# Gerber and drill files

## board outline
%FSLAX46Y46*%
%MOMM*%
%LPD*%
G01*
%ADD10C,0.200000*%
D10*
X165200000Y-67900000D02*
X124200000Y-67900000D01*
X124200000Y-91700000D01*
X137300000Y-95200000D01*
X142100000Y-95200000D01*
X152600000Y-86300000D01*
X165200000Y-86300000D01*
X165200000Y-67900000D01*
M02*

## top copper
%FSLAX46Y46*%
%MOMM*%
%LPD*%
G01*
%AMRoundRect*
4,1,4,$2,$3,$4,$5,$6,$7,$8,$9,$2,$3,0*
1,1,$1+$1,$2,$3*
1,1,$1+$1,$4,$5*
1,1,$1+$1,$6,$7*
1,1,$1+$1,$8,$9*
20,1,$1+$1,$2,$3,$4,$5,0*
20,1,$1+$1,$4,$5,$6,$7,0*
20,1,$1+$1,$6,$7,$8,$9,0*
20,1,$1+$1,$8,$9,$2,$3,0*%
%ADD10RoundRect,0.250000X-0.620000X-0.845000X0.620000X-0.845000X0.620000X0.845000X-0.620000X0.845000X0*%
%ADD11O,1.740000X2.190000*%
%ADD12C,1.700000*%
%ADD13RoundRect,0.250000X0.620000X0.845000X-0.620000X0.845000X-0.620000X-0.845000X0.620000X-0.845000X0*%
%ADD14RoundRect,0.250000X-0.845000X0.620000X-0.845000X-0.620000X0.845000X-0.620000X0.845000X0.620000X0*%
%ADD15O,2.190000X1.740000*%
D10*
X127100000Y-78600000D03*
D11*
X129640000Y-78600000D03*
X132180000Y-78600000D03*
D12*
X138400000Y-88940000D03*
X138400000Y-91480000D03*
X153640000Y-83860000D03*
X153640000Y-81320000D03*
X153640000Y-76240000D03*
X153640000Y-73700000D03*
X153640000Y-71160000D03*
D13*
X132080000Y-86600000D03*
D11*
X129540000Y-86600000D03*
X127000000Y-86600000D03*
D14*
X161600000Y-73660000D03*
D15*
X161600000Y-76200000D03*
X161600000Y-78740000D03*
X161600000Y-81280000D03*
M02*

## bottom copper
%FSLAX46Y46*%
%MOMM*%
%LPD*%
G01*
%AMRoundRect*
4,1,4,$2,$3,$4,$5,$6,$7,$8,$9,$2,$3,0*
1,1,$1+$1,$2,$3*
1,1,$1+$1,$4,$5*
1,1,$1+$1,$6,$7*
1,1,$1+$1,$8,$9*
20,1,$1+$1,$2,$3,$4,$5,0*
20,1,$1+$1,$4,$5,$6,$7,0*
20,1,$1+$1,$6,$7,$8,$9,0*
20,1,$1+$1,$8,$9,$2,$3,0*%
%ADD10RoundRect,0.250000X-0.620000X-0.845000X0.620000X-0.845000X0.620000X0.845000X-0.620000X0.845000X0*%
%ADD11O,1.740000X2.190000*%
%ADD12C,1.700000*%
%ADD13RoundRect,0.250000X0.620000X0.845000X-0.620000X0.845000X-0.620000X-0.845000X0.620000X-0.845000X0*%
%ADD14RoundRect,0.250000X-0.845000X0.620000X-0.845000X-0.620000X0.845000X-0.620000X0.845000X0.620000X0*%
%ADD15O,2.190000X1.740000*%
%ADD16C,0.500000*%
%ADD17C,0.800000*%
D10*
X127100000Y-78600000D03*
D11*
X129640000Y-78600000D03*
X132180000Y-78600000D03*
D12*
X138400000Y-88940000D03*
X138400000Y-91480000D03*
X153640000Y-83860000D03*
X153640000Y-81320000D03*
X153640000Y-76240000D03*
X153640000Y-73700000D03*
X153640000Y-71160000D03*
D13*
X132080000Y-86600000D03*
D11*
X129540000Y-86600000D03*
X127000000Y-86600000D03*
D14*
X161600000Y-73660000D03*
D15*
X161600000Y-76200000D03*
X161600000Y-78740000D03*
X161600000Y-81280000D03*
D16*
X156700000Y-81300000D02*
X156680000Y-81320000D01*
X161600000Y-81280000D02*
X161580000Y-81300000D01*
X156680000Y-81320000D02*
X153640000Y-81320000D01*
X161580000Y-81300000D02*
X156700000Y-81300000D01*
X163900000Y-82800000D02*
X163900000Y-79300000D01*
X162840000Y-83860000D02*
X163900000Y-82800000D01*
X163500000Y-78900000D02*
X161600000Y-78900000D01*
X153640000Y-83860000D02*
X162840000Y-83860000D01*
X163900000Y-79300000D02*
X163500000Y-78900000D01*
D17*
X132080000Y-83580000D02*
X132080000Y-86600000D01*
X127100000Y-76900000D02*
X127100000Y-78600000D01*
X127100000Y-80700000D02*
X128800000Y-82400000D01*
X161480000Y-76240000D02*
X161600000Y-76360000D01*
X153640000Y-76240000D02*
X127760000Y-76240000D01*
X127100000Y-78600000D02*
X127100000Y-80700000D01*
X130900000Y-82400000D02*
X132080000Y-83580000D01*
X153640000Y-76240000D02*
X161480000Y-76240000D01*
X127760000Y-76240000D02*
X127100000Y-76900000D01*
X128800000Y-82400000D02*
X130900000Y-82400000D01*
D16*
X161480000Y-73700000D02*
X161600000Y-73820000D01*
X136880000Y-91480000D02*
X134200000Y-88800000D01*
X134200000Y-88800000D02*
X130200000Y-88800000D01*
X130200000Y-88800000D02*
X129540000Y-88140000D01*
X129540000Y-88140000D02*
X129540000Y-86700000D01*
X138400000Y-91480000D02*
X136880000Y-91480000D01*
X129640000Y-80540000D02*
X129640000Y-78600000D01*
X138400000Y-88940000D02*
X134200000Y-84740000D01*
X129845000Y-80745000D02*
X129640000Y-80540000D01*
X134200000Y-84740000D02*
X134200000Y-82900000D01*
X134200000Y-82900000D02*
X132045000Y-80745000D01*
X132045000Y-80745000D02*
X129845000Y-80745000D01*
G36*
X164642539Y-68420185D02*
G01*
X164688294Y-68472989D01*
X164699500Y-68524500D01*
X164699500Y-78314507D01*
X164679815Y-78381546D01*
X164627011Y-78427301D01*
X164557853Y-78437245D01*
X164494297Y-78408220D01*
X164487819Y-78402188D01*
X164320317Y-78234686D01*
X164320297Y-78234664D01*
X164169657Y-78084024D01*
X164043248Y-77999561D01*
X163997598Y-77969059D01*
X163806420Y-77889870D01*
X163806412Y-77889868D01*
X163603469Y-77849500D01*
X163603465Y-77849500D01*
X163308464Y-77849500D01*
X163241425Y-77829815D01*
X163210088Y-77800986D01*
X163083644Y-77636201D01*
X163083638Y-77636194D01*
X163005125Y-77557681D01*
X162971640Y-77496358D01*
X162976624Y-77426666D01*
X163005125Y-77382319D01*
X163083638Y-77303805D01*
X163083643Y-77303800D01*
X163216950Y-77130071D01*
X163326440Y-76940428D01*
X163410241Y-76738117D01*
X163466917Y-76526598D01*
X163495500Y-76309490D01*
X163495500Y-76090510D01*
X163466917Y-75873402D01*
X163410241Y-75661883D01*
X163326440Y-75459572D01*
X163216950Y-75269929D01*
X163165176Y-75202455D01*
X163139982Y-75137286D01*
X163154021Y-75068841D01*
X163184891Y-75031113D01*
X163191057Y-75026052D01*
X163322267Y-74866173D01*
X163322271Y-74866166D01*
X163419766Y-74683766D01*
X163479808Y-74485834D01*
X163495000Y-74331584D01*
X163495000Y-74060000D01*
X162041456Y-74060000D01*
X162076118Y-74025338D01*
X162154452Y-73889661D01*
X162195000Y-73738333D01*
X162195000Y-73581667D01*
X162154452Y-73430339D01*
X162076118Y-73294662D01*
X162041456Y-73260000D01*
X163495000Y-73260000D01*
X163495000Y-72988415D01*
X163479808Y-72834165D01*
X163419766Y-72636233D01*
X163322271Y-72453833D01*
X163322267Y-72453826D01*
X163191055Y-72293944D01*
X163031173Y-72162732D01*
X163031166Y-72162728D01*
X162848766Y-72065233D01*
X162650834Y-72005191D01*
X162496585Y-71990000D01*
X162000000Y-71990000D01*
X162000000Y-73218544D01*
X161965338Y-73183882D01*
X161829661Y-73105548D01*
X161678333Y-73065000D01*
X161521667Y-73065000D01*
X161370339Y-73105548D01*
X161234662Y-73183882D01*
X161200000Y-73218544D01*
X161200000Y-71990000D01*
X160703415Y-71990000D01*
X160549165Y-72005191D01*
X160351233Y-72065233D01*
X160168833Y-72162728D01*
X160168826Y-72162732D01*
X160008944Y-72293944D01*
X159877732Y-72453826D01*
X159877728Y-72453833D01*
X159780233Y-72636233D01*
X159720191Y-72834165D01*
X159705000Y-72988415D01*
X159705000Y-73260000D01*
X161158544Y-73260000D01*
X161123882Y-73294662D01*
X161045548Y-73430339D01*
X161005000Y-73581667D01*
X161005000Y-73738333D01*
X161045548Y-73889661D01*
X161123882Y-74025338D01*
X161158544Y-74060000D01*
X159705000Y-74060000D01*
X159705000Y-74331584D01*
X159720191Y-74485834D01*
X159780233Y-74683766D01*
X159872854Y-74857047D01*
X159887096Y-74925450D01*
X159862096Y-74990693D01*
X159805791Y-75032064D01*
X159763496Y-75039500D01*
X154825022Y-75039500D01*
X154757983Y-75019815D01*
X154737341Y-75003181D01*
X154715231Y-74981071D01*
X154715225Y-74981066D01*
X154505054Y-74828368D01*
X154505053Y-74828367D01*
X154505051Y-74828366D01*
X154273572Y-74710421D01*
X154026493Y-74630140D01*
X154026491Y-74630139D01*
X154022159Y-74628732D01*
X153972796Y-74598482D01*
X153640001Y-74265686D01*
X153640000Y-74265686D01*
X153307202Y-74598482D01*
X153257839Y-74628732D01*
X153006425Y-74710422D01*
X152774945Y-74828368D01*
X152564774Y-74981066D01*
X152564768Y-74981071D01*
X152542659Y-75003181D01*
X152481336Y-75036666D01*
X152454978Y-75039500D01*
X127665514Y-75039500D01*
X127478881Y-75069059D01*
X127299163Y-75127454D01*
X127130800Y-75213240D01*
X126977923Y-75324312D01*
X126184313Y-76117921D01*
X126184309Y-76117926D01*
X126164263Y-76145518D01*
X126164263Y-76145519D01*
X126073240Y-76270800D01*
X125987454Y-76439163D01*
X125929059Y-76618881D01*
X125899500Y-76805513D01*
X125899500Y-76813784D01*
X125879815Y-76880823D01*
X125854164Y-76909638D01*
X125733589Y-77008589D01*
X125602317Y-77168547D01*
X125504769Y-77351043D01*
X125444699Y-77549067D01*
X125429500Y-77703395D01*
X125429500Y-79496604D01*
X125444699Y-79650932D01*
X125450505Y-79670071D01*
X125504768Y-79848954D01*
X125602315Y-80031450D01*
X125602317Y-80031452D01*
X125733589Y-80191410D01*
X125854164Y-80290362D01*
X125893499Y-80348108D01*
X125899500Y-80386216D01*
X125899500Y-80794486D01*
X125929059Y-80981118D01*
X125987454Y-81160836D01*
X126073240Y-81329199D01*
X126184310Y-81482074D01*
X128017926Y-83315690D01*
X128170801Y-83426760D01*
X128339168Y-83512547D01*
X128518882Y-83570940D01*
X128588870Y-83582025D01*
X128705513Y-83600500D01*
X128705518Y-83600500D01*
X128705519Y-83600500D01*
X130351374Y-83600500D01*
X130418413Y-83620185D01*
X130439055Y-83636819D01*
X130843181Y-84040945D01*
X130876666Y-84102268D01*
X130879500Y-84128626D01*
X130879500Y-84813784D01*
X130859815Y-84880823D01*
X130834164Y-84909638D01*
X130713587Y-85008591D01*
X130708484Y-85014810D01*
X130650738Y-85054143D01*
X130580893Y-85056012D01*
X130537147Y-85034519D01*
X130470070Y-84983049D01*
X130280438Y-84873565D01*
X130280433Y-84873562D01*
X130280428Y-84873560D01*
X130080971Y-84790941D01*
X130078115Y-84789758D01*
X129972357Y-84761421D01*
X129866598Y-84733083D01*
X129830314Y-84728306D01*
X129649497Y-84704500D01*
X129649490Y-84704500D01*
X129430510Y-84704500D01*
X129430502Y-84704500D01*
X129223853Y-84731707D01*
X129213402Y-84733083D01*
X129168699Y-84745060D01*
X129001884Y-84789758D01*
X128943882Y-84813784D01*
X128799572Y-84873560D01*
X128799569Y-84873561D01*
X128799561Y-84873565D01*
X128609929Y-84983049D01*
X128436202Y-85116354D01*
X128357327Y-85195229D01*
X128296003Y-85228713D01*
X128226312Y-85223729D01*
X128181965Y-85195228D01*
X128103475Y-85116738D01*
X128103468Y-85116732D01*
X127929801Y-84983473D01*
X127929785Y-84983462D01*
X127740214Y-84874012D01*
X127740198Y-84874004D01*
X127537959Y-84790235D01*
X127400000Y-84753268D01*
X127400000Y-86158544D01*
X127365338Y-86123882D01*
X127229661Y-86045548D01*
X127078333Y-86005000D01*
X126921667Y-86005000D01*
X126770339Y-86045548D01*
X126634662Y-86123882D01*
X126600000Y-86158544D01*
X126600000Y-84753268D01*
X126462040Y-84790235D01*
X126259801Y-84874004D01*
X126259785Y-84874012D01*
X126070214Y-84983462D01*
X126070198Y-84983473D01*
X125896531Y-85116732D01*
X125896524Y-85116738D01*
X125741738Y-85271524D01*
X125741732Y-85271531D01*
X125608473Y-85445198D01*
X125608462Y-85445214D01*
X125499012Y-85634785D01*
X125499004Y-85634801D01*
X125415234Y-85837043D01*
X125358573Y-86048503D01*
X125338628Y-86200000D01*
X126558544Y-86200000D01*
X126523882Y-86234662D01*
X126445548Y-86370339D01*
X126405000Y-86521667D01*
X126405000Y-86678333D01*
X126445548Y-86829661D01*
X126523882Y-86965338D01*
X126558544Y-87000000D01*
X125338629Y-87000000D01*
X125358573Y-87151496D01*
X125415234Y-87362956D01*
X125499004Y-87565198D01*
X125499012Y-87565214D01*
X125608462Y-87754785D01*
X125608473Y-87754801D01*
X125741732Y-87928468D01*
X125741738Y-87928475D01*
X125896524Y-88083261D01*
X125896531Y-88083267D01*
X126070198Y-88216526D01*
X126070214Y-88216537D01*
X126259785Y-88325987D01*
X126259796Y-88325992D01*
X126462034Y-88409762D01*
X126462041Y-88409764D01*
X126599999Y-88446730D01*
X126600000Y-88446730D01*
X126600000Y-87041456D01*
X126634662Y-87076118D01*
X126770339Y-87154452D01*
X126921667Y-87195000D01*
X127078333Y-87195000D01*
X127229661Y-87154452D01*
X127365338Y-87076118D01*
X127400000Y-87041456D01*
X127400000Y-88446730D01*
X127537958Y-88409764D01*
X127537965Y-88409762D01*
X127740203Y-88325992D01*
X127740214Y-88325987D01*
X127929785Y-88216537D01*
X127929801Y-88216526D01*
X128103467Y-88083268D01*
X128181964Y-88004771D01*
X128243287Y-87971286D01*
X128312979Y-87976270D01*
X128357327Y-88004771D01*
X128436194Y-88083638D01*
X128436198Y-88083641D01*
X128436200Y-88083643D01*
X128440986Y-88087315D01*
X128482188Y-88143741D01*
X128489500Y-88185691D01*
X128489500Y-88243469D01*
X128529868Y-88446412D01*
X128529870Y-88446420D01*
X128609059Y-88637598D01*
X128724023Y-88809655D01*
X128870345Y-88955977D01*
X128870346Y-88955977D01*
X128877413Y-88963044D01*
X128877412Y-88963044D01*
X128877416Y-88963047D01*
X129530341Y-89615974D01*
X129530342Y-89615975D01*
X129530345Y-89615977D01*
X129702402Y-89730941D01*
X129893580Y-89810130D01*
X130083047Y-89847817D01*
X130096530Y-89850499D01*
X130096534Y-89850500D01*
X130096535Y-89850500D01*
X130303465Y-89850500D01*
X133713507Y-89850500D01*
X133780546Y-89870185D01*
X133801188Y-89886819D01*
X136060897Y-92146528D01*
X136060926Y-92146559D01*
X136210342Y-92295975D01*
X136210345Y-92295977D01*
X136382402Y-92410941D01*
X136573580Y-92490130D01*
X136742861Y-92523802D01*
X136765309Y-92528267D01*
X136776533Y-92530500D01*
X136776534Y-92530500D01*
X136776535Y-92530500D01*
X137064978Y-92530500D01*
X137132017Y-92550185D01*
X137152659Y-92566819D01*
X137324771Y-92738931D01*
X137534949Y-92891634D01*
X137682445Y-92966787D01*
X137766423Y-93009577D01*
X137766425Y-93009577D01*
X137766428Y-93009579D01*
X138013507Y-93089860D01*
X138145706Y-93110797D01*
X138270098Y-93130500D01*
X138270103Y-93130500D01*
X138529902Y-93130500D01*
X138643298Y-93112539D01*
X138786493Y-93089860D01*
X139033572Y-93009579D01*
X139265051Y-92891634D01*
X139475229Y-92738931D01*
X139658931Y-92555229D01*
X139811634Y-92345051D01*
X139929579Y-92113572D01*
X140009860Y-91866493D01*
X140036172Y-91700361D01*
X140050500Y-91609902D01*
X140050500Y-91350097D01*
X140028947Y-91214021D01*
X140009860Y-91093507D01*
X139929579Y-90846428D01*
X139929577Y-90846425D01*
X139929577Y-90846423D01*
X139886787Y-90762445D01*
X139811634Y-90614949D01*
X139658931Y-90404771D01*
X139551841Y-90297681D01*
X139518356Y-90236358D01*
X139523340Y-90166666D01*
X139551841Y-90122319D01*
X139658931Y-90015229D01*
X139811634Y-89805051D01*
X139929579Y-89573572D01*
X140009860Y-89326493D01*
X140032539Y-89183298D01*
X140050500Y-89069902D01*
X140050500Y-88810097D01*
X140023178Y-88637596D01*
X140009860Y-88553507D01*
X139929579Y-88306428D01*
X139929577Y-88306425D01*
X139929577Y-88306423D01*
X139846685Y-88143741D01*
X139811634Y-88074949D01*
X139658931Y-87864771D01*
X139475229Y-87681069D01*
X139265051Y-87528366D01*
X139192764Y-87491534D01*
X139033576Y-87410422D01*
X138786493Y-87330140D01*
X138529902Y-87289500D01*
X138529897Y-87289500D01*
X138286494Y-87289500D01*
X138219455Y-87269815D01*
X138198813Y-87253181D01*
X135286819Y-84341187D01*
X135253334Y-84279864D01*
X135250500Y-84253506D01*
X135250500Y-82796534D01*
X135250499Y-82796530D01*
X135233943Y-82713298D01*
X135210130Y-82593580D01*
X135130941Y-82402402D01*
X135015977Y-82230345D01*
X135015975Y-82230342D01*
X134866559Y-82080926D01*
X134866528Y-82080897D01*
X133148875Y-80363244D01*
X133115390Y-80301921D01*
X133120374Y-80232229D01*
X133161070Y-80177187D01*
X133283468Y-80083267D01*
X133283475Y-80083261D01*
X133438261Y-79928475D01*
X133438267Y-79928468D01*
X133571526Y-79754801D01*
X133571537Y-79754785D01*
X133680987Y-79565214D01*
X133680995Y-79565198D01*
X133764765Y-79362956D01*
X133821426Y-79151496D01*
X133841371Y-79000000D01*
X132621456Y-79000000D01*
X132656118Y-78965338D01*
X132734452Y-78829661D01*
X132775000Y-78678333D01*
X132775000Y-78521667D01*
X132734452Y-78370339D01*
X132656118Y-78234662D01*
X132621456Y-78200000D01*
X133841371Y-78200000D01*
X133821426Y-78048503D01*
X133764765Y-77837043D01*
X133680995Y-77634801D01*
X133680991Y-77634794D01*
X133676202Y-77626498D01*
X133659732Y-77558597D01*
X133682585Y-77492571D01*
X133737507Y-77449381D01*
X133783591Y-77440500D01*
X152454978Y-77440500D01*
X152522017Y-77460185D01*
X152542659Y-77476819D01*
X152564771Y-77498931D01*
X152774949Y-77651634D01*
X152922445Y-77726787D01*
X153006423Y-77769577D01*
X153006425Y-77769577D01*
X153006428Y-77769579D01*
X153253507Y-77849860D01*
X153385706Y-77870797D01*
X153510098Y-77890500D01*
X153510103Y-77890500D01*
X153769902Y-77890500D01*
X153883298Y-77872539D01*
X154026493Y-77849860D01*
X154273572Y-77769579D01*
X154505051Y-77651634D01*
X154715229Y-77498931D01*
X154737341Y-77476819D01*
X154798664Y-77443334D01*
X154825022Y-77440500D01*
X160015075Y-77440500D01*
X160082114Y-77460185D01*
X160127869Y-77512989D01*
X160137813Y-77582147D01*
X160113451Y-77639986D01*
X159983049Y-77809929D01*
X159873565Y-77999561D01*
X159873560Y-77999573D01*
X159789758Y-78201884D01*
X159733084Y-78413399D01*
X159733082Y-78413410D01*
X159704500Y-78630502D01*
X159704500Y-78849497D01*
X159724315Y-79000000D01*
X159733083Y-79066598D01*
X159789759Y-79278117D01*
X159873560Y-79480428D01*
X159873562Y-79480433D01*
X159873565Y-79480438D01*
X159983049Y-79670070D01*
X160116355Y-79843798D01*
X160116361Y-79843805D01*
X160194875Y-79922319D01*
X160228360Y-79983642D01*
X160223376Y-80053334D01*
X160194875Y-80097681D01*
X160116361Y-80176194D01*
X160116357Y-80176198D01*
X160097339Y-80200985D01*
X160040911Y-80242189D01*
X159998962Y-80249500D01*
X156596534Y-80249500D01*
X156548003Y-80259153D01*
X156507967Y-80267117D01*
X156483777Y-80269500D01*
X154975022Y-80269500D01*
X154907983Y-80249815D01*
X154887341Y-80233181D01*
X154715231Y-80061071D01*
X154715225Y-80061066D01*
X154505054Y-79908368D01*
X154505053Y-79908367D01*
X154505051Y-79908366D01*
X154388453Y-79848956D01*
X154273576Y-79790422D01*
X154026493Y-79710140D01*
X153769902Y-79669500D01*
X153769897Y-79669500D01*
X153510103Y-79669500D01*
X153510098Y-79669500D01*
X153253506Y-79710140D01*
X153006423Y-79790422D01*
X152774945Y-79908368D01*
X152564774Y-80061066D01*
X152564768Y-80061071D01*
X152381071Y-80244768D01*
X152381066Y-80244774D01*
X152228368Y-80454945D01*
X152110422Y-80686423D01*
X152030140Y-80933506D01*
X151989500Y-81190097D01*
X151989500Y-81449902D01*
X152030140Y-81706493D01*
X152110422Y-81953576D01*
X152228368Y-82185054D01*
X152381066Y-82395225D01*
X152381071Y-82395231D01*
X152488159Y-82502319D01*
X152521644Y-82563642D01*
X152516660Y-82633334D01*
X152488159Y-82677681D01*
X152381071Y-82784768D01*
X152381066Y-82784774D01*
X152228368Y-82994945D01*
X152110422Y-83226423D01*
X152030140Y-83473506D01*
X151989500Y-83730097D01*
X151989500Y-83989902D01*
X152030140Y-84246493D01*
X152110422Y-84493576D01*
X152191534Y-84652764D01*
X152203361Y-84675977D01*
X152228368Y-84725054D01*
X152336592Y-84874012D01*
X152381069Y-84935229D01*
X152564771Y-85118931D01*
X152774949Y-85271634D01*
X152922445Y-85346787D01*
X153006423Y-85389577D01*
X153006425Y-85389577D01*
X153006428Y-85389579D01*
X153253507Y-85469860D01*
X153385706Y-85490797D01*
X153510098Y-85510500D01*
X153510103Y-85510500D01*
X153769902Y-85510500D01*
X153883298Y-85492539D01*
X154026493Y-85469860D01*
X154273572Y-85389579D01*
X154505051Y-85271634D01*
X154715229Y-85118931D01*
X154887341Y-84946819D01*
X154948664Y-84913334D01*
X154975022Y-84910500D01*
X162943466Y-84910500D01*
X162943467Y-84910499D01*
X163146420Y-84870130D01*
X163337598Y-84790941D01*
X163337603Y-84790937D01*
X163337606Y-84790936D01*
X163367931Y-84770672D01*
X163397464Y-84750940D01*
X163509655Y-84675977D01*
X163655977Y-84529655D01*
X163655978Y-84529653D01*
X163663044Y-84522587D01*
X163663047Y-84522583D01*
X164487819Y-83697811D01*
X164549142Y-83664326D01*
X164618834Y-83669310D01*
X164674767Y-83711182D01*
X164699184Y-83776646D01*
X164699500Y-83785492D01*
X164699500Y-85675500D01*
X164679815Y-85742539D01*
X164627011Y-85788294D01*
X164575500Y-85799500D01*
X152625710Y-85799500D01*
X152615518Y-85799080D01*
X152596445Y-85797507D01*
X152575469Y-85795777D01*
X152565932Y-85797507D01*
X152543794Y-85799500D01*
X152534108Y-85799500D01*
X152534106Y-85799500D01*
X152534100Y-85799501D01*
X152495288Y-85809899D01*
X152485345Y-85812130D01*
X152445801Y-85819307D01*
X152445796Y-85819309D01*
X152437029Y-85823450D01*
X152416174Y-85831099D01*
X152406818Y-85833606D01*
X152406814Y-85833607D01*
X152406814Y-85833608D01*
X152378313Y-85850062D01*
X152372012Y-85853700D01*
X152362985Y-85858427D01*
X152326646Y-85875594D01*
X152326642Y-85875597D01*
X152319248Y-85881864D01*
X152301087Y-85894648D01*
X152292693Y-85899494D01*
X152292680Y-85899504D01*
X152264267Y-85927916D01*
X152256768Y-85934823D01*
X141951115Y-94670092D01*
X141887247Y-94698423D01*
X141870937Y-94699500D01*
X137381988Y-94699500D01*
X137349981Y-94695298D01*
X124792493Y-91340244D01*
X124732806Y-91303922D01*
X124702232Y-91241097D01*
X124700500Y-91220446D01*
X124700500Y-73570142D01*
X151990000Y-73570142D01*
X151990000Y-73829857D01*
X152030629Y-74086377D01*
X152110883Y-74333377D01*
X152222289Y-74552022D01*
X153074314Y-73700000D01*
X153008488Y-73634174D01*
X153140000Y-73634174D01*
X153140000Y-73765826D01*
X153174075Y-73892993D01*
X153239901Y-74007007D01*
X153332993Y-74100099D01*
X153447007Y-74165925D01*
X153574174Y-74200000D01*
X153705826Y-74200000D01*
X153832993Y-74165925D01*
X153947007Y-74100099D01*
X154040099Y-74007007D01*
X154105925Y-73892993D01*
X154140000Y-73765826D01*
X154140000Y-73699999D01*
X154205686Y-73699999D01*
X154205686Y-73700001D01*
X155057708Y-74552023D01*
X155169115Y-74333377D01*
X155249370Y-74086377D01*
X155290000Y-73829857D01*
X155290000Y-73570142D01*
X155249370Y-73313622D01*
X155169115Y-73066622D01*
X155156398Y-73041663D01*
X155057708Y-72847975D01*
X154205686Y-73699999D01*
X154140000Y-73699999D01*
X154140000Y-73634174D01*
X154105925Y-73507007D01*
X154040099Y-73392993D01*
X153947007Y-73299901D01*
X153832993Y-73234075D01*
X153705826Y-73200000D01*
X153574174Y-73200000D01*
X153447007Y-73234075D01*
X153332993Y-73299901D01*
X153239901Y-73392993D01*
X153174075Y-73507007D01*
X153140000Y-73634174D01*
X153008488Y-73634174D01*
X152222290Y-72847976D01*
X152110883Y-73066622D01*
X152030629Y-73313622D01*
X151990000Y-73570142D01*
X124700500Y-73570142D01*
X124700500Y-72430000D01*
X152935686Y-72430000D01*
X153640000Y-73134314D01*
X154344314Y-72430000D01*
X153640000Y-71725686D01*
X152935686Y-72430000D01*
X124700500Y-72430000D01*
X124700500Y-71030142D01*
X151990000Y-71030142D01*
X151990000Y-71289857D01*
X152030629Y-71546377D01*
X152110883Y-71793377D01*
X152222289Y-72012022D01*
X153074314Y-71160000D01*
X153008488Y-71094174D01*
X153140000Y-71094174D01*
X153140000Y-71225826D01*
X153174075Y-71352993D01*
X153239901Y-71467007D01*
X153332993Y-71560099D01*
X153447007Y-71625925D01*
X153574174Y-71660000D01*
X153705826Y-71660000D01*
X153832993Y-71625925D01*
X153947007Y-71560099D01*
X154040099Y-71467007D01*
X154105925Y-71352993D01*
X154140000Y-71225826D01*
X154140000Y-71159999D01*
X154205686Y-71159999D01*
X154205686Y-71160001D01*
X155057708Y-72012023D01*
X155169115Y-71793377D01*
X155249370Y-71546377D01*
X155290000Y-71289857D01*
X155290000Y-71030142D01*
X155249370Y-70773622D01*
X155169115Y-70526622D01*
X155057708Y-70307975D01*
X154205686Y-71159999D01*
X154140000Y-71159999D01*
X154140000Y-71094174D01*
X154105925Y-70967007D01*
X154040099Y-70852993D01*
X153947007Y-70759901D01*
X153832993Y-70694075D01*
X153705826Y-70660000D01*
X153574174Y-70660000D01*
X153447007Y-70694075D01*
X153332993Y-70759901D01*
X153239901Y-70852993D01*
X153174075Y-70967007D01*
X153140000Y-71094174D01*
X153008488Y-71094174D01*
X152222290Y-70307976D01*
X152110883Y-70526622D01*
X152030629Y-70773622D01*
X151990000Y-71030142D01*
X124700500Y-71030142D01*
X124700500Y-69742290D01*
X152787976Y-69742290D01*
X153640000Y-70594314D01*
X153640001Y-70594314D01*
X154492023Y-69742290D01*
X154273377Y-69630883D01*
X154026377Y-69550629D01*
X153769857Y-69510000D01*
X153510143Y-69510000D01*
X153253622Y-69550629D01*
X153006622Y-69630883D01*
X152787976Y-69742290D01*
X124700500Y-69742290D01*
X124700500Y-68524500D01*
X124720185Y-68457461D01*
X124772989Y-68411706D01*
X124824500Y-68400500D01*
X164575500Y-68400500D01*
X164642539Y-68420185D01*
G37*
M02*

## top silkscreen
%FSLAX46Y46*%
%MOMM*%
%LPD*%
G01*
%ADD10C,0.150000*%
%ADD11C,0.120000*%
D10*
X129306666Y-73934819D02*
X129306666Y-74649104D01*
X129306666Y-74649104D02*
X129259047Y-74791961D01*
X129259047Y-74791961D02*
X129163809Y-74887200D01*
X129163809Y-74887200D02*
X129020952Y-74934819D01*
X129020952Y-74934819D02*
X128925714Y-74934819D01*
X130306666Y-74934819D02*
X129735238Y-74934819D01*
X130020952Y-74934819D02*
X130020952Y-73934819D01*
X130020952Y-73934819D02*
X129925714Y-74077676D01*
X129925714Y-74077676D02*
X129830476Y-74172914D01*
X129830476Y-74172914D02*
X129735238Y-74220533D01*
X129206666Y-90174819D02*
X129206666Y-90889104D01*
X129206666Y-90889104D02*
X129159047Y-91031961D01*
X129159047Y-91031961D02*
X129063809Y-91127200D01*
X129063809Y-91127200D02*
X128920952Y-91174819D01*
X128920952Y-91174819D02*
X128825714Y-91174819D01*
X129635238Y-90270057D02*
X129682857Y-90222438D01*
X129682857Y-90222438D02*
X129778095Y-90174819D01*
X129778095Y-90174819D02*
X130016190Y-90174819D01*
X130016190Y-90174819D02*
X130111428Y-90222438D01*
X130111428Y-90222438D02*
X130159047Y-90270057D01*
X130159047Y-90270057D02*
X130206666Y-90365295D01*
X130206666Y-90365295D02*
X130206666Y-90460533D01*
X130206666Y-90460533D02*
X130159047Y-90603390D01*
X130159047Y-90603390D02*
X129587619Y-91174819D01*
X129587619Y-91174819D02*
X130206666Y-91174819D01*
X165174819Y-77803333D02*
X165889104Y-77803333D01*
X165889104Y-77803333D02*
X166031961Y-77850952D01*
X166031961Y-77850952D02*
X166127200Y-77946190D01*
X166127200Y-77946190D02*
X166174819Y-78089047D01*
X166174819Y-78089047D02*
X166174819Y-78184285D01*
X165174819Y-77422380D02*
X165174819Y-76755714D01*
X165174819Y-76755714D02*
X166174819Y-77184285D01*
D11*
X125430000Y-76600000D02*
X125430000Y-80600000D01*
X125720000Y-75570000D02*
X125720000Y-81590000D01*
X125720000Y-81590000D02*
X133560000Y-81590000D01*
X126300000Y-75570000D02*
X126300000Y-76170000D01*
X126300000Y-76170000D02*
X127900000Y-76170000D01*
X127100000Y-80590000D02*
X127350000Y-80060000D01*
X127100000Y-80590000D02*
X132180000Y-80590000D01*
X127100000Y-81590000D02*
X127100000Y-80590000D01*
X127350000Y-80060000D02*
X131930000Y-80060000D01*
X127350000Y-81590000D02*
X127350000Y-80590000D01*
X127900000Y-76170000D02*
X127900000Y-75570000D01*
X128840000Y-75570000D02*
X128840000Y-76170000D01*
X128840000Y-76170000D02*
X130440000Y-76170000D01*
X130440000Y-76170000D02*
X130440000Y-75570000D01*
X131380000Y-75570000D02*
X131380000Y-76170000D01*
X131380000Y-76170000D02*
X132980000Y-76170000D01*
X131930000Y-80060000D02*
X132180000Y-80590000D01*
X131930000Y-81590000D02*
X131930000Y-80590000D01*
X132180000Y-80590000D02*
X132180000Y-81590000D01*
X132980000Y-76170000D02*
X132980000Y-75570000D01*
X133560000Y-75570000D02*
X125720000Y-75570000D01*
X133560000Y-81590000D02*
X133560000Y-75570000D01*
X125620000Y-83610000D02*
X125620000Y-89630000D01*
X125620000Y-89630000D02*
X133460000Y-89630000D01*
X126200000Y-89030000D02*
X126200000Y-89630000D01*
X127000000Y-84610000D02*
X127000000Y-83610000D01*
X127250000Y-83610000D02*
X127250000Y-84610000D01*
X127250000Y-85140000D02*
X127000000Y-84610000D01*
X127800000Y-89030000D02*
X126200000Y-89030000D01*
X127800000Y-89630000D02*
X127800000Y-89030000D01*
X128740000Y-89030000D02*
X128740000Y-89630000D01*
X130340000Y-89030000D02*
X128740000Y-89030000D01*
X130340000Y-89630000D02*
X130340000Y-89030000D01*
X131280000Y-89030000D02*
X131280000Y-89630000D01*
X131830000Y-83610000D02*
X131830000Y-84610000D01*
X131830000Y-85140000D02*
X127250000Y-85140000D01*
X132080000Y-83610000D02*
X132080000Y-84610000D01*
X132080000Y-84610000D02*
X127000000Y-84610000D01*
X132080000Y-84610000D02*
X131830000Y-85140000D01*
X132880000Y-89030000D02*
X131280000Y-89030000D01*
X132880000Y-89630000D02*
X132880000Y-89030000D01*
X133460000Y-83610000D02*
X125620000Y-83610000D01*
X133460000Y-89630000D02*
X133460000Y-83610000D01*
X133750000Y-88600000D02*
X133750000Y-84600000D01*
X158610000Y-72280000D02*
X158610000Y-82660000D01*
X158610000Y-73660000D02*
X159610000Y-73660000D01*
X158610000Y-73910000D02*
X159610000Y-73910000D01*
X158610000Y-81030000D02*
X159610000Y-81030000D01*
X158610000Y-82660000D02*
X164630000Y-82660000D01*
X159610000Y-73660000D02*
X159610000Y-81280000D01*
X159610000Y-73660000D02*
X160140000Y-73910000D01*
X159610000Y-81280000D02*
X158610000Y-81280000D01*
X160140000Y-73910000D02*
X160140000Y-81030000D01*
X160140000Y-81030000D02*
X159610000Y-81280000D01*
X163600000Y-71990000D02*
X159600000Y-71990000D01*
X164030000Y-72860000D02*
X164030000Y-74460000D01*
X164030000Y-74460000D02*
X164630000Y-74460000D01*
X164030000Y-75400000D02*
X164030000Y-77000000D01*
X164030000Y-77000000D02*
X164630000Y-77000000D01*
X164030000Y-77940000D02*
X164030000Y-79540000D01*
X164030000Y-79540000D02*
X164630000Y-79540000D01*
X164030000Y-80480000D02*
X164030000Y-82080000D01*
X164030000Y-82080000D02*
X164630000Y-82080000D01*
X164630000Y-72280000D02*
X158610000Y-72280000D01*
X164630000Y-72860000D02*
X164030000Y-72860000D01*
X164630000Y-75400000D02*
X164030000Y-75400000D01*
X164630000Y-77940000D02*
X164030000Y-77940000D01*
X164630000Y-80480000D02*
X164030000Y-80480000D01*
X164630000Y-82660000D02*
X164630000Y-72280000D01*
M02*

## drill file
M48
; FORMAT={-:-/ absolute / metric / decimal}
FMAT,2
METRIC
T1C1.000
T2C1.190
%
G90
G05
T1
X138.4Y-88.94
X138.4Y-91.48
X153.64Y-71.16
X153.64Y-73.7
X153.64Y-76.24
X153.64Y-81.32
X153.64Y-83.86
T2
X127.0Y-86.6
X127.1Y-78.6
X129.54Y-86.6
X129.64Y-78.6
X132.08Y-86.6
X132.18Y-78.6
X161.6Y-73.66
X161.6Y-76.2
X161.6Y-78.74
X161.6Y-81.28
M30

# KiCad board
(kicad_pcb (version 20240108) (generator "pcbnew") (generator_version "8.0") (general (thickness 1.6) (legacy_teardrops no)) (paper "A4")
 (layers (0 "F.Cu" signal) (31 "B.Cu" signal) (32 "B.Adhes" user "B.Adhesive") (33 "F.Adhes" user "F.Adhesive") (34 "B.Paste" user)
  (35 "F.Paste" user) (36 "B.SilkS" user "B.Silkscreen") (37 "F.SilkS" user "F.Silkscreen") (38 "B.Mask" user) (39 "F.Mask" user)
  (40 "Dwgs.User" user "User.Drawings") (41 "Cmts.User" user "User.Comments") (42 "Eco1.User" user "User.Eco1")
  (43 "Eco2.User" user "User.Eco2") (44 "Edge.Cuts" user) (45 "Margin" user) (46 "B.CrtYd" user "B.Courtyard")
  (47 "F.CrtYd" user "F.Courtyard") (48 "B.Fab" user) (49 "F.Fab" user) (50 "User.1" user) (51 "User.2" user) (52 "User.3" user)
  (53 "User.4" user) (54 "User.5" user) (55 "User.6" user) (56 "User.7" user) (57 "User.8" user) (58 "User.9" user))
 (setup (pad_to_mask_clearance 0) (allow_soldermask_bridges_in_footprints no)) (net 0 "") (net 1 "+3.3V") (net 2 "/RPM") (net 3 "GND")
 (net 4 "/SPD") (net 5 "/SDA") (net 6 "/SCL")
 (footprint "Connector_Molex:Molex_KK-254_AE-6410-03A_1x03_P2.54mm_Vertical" (layer "F.Cu") (at 127.1 78.6)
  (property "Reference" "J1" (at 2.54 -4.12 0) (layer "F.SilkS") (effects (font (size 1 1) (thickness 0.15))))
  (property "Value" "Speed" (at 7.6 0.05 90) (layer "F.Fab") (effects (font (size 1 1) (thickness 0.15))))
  (fp_line (start -1.67 -2) (end -1.67 2) (stroke (width 0.12) (type solid)) (layer "F.SilkS"))
  (fp_line (start -1.38 -3.03) (end -1.38 2.99) (stroke (width 0.12) (type solid)) (layer "F.SilkS"))
  (fp_line (start -1.38 2.99) (end 6.46 2.99) (stroke (width 0.12) (type solid)) (layer "F.SilkS"))
  (fp_line (start -0.8 -3.03) (end -0.8 -2.43) (stroke (width 0.12) (type solid)) (layer "F.SilkS"))
  (fp_line (start -0.8 -2.43) (end 0.8 -2.43) (stroke (width 0.12) (type solid)) (layer "F.SilkS"))
  (fp_line (start 0 1.99) (end 0.25 1.46) (stroke (width 0.12) (type solid)) (layer "F.SilkS"))
  (fp_line (start 0 1.99) (end 5.08 1.99) (stroke (width 0.12) (type solid)) (layer "F.SilkS"))
  (fp_line (start 0 2.99) (end 0 1.99) (stroke (width 0.12) (type solid)) (layer "F.SilkS"))
  (fp_line (start 0.25 1.46) (end 4.83 1.46) (stroke (width 0.12) (type solid)) (layer "F.SilkS"))
  (fp_line (start 0.25 2.99) (end 0.25 1.99) (stroke (width 0.12) (type solid)) (layer "F.SilkS"))
  (fp_line (start 0.8 -2.43) (end 0.8 -3.03) (stroke (width 0.12) (type solid)) (layer "F.SilkS"))
  (fp_line (start 1.74 -3.03) (end 1.74 -2.43) (stroke (width 0.12) (type solid)) (layer "F.SilkS"))
  (fp_line (start 1.74 -2.43) (end 3.34 -2.43) (stroke (width 0.12) (type solid)) (layer "F.SilkS"))
  (fp_line (start 3.34 -2.43) (end 3.34 -3.03) (stroke (width 0.12) (type solid)) (layer "F.SilkS"))
  (fp_line (start 4.28 -3.03) (end 4.28 -2.43) (stroke (width 0.12) (type solid)) (layer "F.SilkS"))
  (fp_line (start 4.28 -2.43) (end 5.88 -2.43) (stroke (width 0.12) (type solid)) (layer "F.SilkS"))
  (fp_line (start 4.83 1.46) (end 5.08 1.99) (stroke (width 0.12) (type solid)) (layer "F.SilkS"))
  (fp_line (start 4.83 2.99) (end 4.83 1.99) (stroke (width 0.12) (type solid)) (layer "F.SilkS"))
  (fp_line (start 5.08 1.99) (end 5.08 2.99) (stroke (width 0.12) (type solid)) (layer "F.SilkS"))
  (fp_line (start 5.88 -2.43) (end 5.88 -3.03) (stroke (width 0.12) (type solid)) (layer "F.SilkS"))
  (fp_line (start 6.46 -3.03) (end -1.38 -3.03) (stroke (width 0.12) (type solid)) (layer "F.SilkS"))
  (fp_line (start 6.46 2.99) (end 6.46 -3.03) (stroke (width 0.12) (type solid)) (layer "F.SilkS"))
  (pad "1" thru_hole roundrect (at 0 0) (size 1.74 2.19) (drill 1.19) (layers "*.Cu" "*.Mask") (remove_unused_layers no)
   (roundrect_rratio 0.143678) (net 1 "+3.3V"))
  (pad "2" thru_hole oval (at 2.54 0) (size 1.74 2.19) (drill 1.19) (layers "*.Cu" "*.Mask") (remove_unused_layers no) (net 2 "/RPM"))
  (pad "3" thru_hole oval (at 5.08 0) (size 1.74 2.19) (drill 1.19) (layers "*.Cu" "*.Mask") (remove_unused_layers no) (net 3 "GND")))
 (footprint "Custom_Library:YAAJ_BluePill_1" (layer "F.Cu") (at 138.4 71.16)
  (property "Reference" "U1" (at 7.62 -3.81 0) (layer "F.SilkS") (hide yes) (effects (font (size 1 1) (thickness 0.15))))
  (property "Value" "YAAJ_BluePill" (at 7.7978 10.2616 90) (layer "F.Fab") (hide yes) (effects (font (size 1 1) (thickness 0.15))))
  (pad "8" thru_hole circle (at 0 17.78) (size 1.7 1.7) (drill 1) (layers "*.Cu" "*.Mask") (remove_unused_layers no) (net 2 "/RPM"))
  (pad "9" thru_hole circle (at 0 20.32) (size 1.7 1.7) (drill 1) (layers "*.Cu" "*.Mask") (remove_unused_layers no) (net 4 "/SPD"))
  (pad "35" thru_hole circle (at 15.24 12.7) (size 1.7 1.7) (drill 1) (layers "*.Cu" "*.Mask") (remove_unused_layers no) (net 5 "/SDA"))
  (pad "36" thru_hole circle (at 15.24 10.16) (size 1.7 1.7) (drill 1) (layers "*.Cu" "*.Mask") (remove_unused_layers no) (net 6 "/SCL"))
  (pad "38" thru_hole circle (at 15.24 5.08) (size 1.7 1.7) (drill 1) (layers "*.Cu" "*.Mask") (remove_unused_layers no) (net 1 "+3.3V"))
  (pad "39" thru_hole circle (at 15.24 2.54) (size 1.7 1.7) (drill 1) (layers "*.Cu" "*.Mask") (remove_unused_layers no) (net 3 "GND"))
  (pad "40" thru_hole circle (at 15.24 0) (size 1.7 1.7) (drill 1) (layers "*.Cu" "*.Mask") (remove_unused_layers no) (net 3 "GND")))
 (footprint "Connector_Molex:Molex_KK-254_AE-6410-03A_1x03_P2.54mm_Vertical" (layer "F.Cu") (at 132.08 86.6 180)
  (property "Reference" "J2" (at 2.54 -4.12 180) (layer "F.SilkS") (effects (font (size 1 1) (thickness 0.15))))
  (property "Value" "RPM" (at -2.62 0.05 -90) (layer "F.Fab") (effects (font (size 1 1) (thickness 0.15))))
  (fp_line (start 6.46 2.99) (end 6.46 -3.03) (stroke (width 0.12) (type solid)) (layer "F.SilkS"))
  (fp_line (start 6.46 -3.03) (end -1.38 -3.03) (stroke (width 0.12) (type solid)) (layer "F.SilkS"))
  (fp_line (start 5.88 -2.43) (end 5.88 -3.03) (stroke (width 0.12) (type solid)) (layer "F.SilkS"))
  (fp_line (start 5.08 1.99) (end 5.08 2.99) (stroke (width 0.12) (type solid)) (layer "F.SilkS"))
  (fp_line (start 4.83 2.99) (end 4.83 1.99) (stroke (width 0.12) (type solid)) (layer "F.SilkS"))
  (fp_line (start 4.83 1.46) (end 5.08 1.99) (stroke (width 0.12) (type solid)) (layer "F.SilkS"))
  (fp_line (start 4.28 -2.43) (end 5.88 -2.43) (stroke (width 0.12) (type solid)) (layer "F.SilkS"))
  (fp_line (start 4.28 -3.03) (end 4.28 -2.43) (stroke (width 0.12) (type solid)) (layer "F.SilkS"))
  (fp_line (start 3.34 -2.43) (end 3.34 -3.03) (stroke (width 0.12) (type solid)) (layer "F.SilkS"))
  (fp_line (start 1.74 -2.43) (end 3.34 -2.43) (stroke (width 0.12) (type solid)) (layer "F.SilkS"))
  (fp_line (start 1.74 -3.03) (end 1.74 -2.43) (stroke (width 0.12) (type solid)) (layer "F.SilkS"))
  (fp_line (start 0.8 -2.43) (end 0.8 -3.03) (stroke (width 0.12) (type solid)) (layer "F.SilkS"))
  (fp_line (start 0.25 2.99) (end 0.25 1.99) (stroke (width 0.12) (type solid)) (layer "F.SilkS"))
  (fp_line (start 0.25 1.46) (end 4.83 1.46) (stroke (width 0.12) (type solid)) (layer "F.SilkS"))
  (fp_line (start 0 2.99) (end 0 1.99) (stroke (width 0.12) (type solid)) (layer "F.SilkS"))
  (fp_line (start 0 1.99) (end 5.08 1.99) (stroke (width 0.12) (type solid)) (layer "F.SilkS"))
  (fp_line (start 0 1.99) (end 0.25 1.46) (stroke (width 0.12) (type solid)) (layer "F.SilkS"))
  (fp_line (start -0.8 -2.43) (end 0.8 -2.43) (stroke (width 0.12) (type solid)) (layer "F.SilkS"))
  (fp_line (start -0.8 -3.03) (end -0.8 -2.43) (stroke (width 0.12) (type solid)) (layer "F.SilkS"))
  (fp_line (start -1.38 2.99) (end 6.46 2.99) (stroke (width 0.12) (type solid)) (layer "F.SilkS"))
  (fp_line (start -1.38 -3.03) (end -1.38 2.99) (stroke (width 0.12) (type solid)) (layer "F.SilkS"))
  (fp_line (start -1.67 -2) (end -1.67 2) (stroke (width 0.12) (type solid)) (layer "F.SilkS"))
  (pad "1" thru_hole roundrect (at 0 0 180) (size 1.74 2.19) (drill 1.19) (layers "*.Cu" "*.Mask") (remove_unused_layers no)
   (roundrect_rratio 0.143678) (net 1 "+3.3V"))
  (pad "2" thru_hole oval (at 2.54 0 180) (size 1.74 2.19) (drill 1.19) (layers "*.Cu" "*.Mask") (remove_unused_layers no) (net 4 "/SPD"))
  (pad "3" thru_hole oval (at 5.08 0 180) (size 1.74 2.19) (drill 1.19) (layers "*.Cu" "*.Mask") (remove_unused_layers no) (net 3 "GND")))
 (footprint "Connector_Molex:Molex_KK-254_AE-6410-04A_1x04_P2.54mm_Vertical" (layer "F.Cu") (at 161.6 73.66 -90)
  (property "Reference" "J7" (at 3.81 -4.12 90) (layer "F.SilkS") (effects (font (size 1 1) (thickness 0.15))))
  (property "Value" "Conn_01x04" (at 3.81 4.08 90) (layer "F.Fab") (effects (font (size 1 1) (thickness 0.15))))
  (fp_line (start -1.38 2.99) (end 9 2.99) (stroke (width 0.12) (type solid)) (layer "F.SilkS"))
  (fp_line (start 0 2.99) (end 0 1.99) (stroke (width 0.12) (type solid)) (layer "F.SilkS"))
  (fp_line (start 0.25 2.99) (end 0.25 1.99) (stroke (width 0.12) (type solid)) (layer "F.SilkS"))
  (fp_line (start 7.37 2.99) (end 7.37 1.99) (stroke (width 0.12) (type solid)) (layer "F.SilkS"))
  (fp_line (start 9 2.99) (end 9 -3.03) (stroke (width 0.12) (type solid)) (layer "F.SilkS"))
  (fp_line (start 0 1.99) (end 7.62 1.99) (stroke (width 0.12) (type solid)) (layer "F.SilkS"))
  (fp_line (start 0 1.99) (end 0.25 1.46) (stroke (width 0.12) (type solid)) (layer "F.SilkS"))
  (fp_line (start 7.62 1.99) (end 7.62 2.99) (stroke (width 0.12) (type solid)) (layer "F.SilkS"))
  (fp_line (start 0.25 1.46) (end 7.37 1.46) (stroke (width 0.12) (type solid)) (layer "F.SilkS"))
  (fp_line (start 7.37 1.46) (end 7.62 1.99) (stroke (width 0.12) (type solid)) (layer "F.SilkS"))
  (fp_line (start -1.67 -2) (end -1.67 2) (stroke (width 0.12) (type solid)) (layer "F.SilkS"))
  (fp_line (start -0.8 -2.43) (end 0.8 -2.43) (stroke (width 0.12) (type solid)) (layer "F.SilkS"))
  (fp_line (start 0.8 -2.43) (end 0.8 -3.03) (stroke (width 0.12) (type solid)) (layer "F.SilkS"))
  (fp_line (start 1.74 -2.43) (end 3.34 -2.43) (stroke (width 0.12) (type solid)) (layer "F.SilkS"))
  (fp_line (start 3.34 -2.43) (end 3.34 -3.03) (stroke (width 0.12) (type solid)) (layer "F.SilkS"))
  (fp_line (start 4.28 -2.43) (end 5.88 -2.43) (stroke (width 0.12) (type solid)) (layer "F.SilkS"))
  (fp_line (start 5.88 -2.43) (end 5.88 -3.03) (stroke (width 0.12) (type solid)) (layer "F.SilkS"))
  (fp_line (start 6.82 -2.43) (end 8.42 -2.43) (stroke (width 0.12) (type solid)) (layer "F.SilkS"))
  (fp_line (start 8.42 -2.43) (end 8.42 -3.03) (stroke (width 0.12) (type solid)) (layer "F.SilkS"))
  (fp_line (start -1.38 -3.03) (end -1.38 2.99) (stroke (width 0.12) (type solid)) (layer "F.SilkS"))
  (fp_line (start -0.8 -3.03) (end -0.8 -2.43) (stroke (width 0.12) (type solid)) (layer "F.SilkS"))
  (fp_line (start 1.74 -3.03) (end 1.74 -2.43) (stroke (width 0.12) (type solid)) (layer "F.SilkS"))
  (fp_line (start 4.28 -3.03) (end 4.28 -2.43) (stroke (width 0.12) (type solid)) (layer "F.SilkS"))
  (fp_line (start 6.82 -3.03) (end 6.82 -2.43) (stroke (width 0.12) (type solid)) (layer "F.SilkS"))
  (fp_line (start 9 -3.03) (end -1.38 -3.03) (stroke (width 0.12) (type solid)) (layer "F.SilkS"))
  (pad "1" thru_hole roundrect (at 0 0 270) (size 1.74 2.19) (drill 1.19) (layers "*.Cu" "*.Mask") (remove_unused_layers no)
   (roundrect_rratio 0.143678) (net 3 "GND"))
  (pad "2" thru_hole oval (at 2.54 0 270) (size 1.74 2.19) (drill 1.19) (layers "*.Cu" "*.Mask") (remove_unused_layers no) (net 1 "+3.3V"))
  (pad "3" thru_hole oval (at 5.08 0 270) (size 1.74 2.19) (drill 1.19) (layers "*.Cu" "*.Mask") (remove_unused_layers no) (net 5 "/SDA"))
  (pad "4" thru_hole oval (at 7.62 0 270) (size 1.74 2.19) (drill 1.19) (layers "*.Cu" "*.Mask") (remove_unused_layers no) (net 6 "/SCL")))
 (gr_poly
  (pts (xy 165.2 67.9) (xy 124.2 67.9) (xy 124.2 91.7) (xy 137.3 95.2) (xy 142.1 95.2) (xy 152.6 86.3) (xy 165.2 86.3))
  (stroke (width 0.2) (type solid)) (fill none) (layer "Edge.Cuts"))
 (segment (start 156.7 81.3) (end 156.68 81.32) (width 0.5) (layer "B.Cu") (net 6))
 (segment (start 161.6 81.28) (end 161.58 81.3) (width 0.5) (layer "B.Cu") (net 6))
 (segment (start 156.68 81.32) (end 153.64 81.32) (width 0.5) (layer "B.Cu") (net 6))
 (segment (start 161.58 81.3) (end 156.7 81.3) (width 0.5) (layer "B.Cu") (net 6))
 (segment (start 163.9 82.8) (end 163.9 79.3) (width 0.5) (layer "B.Cu") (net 5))
 (segment (start 162.84 83.86) (end 163.9 82.8) (width 0.5) (layer "B.Cu") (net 5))
 (segment (start 163.5 78.9) (end 161.6 78.9) (width 0.5) (layer "B.Cu") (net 5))
 (segment (start 153.64 83.86) (end 162.84 83.86) (width 0.5) (layer "B.Cu") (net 5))
 (segment (start 163.9 79.3) (end 163.5 78.9) (width 0.5) (layer "B.Cu") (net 5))
 (segment (start 132.08 83.58) (end 132.08 86.6) (width 0.8) (layer "B.Cu") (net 1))
 (segment (start 127.1 76.9) (end 127.1 78.6) (width 0.8) (layer "B.Cu") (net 1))
 (segment (start 127.1 80.7) (end 128.8 82.4) (width 0.8) (layer "B.Cu") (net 1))
 (segment (start 161.48 76.24) (end 161.6 76.36) (width 0.8) (layer "B.Cu") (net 1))
 (segment (start 153.64 76.24) (end 127.76 76.24) (width 0.8) (layer "B.Cu") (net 1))
 (segment (start 127.1 78.6) (end 127.1 80.7) (width 0.8) (layer "B.Cu") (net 1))
 (segment (start 130.9 82.4) (end 132.08 83.58) (width 0.8) (layer "B.Cu") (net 1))
 (segment (start 153.64 76.24) (end 161.48 76.24) (width 0.8) (layer "B.Cu") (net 1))
 (segment (start 127.76 76.24) (end 127.1 76.9) (width 0.8) (layer "B.Cu") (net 1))
 (segment (start 128.8 82.4) (end 130.9 82.4) (width 0.8) (layer "B.Cu") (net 1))
 (segment (start 161.48 73.7) (end 161.6 73.82) (width 0.5) (layer "B.Cu") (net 3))
 (segment (start 136.88 91.48) (end 134.2 88.8) (width 0.5) (layer "B.Cu") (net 4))
 (segment (start 134.2 88.8) (end 130.2 88.8) (width 0.5) (layer "B.Cu") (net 4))
 (segment (start 130.2 88.8) (end 129.54 88.14) (width 0.5) (layer "B.Cu") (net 4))
 (segment (start 129.54 88.14) (end 129.54 86.7) (width 0.5) (layer "B.Cu") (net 4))
 (segment (start 138.4 91.48) (end 136.88 91.48) (width 0.5) (layer "B.Cu") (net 4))
 (segment (start 129.64 80.54) (end 129.64 78.6) (width 0.5) (layer "B.Cu") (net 2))
 (segment (start 138.4 88.94) (end 134.2 84.74) (width 0.5) (layer "B.Cu") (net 2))
 (segment (start 129.845 80.745) (end 129.64 80.54) (width 0.5) (layer "B.Cu") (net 2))
 (segment (start 134.2 84.74) (end 134.2 82.9) (width 0.5) (layer "B.Cu") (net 2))
 (segment (start 134.2 82.9) (end 132.045 80.745) (width 0.5) (layer "B.Cu") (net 2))
 (segment (start 132.045 80.745) (end 129.845 80.745) (width 0.5) (layer "B.Cu") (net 2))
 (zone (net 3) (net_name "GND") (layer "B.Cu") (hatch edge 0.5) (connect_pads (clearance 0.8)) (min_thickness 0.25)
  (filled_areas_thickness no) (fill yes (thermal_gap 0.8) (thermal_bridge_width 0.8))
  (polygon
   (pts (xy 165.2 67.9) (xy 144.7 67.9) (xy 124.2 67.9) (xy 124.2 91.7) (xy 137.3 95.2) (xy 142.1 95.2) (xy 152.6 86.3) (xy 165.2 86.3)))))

